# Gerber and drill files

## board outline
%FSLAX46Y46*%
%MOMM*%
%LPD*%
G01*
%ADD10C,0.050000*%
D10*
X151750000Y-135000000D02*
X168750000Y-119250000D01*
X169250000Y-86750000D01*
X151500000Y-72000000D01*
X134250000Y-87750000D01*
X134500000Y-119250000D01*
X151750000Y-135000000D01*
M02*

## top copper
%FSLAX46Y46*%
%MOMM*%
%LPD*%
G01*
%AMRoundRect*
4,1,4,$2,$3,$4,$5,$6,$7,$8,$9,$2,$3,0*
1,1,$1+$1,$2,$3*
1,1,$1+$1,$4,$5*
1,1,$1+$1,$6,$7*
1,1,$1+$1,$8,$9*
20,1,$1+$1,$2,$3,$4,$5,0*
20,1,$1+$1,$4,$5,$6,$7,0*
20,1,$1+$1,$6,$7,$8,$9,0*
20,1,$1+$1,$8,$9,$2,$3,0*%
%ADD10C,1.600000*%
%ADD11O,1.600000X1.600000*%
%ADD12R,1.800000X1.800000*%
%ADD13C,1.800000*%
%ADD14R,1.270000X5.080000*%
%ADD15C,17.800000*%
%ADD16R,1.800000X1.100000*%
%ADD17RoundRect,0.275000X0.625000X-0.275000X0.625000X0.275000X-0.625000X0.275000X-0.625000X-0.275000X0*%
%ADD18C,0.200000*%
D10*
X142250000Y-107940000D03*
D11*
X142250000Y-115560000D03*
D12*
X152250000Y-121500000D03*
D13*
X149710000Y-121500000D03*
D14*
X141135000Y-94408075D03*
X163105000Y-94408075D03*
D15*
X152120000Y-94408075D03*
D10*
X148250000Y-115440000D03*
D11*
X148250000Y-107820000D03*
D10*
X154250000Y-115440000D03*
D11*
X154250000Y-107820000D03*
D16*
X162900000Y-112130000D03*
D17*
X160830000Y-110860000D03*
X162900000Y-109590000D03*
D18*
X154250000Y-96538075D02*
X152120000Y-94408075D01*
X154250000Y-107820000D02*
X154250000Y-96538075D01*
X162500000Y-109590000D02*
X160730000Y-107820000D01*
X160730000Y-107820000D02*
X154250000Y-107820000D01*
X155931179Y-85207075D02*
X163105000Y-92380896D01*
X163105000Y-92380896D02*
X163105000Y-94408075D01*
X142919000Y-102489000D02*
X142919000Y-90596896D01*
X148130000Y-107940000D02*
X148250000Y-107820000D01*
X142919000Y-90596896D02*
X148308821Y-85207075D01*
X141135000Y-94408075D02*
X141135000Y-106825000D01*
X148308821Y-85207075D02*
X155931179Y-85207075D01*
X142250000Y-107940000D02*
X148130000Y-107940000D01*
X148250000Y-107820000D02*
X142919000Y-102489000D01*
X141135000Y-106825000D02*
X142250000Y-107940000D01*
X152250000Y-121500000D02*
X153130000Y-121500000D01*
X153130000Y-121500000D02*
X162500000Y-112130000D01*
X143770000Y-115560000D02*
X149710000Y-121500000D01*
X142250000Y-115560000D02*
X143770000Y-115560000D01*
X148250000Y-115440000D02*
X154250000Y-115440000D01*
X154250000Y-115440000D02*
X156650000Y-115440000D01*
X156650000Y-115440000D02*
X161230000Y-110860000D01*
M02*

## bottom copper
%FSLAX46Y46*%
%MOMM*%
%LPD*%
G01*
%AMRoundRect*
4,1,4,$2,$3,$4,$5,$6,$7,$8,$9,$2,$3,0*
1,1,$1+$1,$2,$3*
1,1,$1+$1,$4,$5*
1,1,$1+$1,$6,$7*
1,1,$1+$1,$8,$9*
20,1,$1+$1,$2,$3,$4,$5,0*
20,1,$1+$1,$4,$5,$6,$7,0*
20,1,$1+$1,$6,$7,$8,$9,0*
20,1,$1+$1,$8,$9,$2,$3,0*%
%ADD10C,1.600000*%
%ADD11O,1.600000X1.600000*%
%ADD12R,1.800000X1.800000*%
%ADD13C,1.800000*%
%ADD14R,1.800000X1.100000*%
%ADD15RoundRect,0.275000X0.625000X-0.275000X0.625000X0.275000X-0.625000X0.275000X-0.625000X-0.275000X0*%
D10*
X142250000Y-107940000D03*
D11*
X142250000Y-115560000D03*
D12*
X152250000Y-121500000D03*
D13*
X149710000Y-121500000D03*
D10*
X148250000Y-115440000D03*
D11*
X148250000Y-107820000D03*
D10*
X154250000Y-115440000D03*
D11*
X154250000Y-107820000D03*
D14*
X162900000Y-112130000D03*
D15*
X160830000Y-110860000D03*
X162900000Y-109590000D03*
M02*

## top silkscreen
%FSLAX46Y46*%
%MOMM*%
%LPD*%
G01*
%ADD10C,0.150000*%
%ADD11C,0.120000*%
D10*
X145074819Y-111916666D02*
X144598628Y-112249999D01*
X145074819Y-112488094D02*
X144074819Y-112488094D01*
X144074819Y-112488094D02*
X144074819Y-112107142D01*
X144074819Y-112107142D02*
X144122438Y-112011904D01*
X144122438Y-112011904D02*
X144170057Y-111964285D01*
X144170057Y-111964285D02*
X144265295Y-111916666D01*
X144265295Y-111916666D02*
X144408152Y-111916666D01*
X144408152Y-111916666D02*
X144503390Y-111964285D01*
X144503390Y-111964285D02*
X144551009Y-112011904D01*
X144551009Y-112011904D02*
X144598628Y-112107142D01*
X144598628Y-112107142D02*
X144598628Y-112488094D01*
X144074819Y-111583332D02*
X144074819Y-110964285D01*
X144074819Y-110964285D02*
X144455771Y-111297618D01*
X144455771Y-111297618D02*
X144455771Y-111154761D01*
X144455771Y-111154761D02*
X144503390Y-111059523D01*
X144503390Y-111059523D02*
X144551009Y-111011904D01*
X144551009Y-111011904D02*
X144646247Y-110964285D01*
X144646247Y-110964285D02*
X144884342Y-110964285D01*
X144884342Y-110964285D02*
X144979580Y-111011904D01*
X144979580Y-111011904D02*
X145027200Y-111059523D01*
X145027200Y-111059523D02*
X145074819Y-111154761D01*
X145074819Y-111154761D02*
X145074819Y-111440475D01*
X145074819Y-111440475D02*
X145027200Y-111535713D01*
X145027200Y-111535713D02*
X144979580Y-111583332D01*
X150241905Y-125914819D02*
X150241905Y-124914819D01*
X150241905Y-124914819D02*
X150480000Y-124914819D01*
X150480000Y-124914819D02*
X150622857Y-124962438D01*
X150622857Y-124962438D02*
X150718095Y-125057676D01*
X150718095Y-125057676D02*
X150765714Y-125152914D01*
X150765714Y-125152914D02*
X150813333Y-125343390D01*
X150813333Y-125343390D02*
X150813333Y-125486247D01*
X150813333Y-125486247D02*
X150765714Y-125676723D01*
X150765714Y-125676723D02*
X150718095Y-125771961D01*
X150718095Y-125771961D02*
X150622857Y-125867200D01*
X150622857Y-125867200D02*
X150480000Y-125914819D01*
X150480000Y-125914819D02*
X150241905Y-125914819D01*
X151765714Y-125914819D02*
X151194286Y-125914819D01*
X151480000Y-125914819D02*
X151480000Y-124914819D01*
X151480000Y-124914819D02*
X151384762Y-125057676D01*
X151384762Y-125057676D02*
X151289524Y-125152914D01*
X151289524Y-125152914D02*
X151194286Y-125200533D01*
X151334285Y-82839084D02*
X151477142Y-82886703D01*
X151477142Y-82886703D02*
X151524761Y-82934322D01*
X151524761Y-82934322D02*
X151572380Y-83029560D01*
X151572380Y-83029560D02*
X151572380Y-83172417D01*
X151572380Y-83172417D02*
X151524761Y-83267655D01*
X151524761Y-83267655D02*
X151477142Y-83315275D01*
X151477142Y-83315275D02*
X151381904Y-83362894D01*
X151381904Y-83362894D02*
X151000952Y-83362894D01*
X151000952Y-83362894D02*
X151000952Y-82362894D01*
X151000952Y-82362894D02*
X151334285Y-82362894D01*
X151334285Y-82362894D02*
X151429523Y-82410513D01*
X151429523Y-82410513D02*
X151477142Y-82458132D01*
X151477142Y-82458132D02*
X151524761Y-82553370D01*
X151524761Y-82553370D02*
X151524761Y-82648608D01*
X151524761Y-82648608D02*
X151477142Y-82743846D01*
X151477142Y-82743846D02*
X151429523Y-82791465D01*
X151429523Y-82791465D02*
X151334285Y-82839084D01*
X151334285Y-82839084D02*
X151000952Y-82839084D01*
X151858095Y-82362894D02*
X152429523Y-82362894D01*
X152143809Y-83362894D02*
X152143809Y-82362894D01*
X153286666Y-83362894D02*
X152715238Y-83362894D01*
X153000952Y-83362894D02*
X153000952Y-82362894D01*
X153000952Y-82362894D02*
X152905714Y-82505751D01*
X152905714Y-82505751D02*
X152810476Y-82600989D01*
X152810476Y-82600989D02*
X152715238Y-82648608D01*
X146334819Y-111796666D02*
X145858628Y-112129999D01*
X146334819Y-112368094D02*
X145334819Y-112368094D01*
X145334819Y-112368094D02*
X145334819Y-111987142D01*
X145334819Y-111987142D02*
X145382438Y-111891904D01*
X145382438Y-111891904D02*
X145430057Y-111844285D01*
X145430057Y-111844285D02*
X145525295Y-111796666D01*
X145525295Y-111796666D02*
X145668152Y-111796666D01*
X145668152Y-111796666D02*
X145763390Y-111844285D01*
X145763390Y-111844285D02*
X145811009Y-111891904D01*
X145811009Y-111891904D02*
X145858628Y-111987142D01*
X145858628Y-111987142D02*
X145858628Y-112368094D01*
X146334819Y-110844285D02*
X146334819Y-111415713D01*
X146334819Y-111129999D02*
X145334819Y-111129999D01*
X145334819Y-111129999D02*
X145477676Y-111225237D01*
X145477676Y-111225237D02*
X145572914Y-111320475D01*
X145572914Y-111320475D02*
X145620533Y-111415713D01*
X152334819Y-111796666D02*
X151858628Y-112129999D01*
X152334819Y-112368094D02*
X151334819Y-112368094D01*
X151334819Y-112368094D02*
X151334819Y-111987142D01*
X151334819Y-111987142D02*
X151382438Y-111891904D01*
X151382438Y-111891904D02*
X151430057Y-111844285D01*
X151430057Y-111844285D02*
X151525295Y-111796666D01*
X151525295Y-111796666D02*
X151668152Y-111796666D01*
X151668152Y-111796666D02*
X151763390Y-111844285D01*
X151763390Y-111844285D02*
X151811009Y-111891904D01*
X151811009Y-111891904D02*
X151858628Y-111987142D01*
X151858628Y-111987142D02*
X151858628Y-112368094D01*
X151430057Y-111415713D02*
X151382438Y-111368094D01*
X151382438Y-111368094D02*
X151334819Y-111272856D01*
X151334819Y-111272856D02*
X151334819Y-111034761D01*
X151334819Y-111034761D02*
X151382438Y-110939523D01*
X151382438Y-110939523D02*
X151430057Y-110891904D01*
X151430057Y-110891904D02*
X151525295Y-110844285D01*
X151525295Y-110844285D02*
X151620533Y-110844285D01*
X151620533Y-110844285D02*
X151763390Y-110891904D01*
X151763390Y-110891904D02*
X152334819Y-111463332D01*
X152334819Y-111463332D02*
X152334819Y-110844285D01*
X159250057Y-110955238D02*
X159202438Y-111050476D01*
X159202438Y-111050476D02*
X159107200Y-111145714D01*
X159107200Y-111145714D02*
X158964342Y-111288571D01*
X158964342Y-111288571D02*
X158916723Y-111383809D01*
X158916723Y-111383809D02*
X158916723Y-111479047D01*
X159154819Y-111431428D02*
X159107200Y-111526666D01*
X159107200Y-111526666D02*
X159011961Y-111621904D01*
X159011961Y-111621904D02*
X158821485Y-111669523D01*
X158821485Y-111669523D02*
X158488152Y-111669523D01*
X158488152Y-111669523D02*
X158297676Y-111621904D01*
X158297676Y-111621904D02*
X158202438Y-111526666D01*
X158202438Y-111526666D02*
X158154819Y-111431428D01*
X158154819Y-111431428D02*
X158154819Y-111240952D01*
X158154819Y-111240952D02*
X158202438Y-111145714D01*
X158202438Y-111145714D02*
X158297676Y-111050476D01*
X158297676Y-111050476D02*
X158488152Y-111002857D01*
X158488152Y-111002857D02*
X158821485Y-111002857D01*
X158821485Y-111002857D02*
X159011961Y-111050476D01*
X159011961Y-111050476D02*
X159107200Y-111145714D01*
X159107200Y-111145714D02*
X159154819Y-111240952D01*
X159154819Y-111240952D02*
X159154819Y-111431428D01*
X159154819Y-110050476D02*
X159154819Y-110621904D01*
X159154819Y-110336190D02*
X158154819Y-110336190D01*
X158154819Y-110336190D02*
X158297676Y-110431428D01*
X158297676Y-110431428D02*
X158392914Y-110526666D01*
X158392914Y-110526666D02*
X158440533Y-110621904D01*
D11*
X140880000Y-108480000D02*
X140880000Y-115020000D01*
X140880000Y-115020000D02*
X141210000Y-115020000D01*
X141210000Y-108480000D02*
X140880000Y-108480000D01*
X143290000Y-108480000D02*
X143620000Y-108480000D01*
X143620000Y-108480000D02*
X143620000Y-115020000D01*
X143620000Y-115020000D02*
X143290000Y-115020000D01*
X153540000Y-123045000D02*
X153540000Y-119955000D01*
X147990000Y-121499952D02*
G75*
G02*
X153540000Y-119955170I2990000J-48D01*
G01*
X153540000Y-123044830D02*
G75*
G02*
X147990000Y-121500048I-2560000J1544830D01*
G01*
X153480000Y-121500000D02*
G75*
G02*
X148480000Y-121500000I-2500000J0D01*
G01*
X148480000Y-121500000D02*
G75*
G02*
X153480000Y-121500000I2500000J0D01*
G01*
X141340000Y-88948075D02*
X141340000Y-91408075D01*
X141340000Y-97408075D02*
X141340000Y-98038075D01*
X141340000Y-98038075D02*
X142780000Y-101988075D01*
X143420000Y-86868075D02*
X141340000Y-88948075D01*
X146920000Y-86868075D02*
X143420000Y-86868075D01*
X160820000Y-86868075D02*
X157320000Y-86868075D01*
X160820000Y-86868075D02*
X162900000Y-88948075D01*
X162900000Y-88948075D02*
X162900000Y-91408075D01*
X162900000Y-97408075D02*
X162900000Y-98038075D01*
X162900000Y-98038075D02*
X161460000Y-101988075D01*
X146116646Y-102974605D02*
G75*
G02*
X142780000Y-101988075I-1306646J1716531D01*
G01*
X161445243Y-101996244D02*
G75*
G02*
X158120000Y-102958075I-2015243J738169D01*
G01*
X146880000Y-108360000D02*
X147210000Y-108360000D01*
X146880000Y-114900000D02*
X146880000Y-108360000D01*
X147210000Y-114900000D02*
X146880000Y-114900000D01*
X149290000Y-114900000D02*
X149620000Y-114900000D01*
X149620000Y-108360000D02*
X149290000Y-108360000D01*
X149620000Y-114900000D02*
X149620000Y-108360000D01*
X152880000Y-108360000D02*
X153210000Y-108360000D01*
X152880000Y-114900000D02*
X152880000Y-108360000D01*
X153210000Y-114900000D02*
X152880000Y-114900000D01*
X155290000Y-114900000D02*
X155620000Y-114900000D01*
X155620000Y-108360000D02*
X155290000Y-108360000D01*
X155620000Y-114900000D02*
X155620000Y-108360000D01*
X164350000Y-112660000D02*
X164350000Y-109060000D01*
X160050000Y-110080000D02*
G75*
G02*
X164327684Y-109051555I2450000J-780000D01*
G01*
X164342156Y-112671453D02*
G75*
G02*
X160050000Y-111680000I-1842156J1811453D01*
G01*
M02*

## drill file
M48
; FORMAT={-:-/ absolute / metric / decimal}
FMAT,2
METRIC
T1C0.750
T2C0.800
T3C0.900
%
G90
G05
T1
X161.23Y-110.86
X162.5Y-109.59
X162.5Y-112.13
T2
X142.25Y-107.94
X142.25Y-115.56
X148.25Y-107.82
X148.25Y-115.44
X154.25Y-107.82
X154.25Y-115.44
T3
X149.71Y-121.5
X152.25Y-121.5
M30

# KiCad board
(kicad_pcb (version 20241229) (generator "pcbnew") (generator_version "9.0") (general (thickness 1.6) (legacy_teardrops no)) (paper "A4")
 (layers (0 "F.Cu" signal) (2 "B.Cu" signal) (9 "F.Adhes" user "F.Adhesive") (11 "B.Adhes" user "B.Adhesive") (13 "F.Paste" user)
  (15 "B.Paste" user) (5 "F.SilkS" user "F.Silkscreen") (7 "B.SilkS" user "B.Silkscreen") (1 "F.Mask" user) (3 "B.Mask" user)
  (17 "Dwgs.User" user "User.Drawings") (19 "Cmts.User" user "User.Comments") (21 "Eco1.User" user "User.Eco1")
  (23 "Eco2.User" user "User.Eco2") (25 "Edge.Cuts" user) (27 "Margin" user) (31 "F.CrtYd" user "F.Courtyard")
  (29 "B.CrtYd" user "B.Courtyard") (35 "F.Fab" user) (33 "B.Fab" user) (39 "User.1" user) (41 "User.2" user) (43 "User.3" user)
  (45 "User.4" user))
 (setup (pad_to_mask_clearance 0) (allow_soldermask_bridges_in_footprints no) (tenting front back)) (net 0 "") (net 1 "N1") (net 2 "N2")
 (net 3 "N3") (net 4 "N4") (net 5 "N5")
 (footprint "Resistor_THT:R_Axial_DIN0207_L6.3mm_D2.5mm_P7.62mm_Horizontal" (layer "F.Cu") (at 142.25 107.94 -90)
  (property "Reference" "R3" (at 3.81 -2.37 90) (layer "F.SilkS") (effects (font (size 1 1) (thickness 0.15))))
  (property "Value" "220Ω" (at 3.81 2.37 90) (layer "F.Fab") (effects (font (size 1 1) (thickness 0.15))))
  (fp_line (start 0.54 1.37) (end 7.08 1.37) (stroke (width 0.12) (type solid)) (layer "F.SilkS"))
  (fp_line (start 7.08 1.37) (end 7.08 1.04) (stroke (width 0.12) (type solid)) (layer "F.SilkS"))
  (fp_line (start 0.54 1.04) (end 0.54 1.37) (stroke (width 0.12) (type solid)) (layer "F.SilkS"))
  (fp_line (start 0.54 -1.04) (end 0.54 -1.37) (stroke (width 0.12) (type solid)) (layer "F.SilkS"))
  (fp_line (start 0.54 -1.37) (end 7.08 -1.37) (stroke (width 0.12) (type solid)) (layer "F.SilkS"))
  (fp_line (start 7.08 -1.37) (end 7.08 -1.04) (stroke (width 0.12) (type solid)) (layer "F.SilkS"))
  (pad "1" thru_hole circle (at 0 0 270) (size 1.6 1.6) (drill 0.8) (layers "*.Cu" "*.Mask") (remove_unused_layers no) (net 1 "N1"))
  (pad "2" thru_hole oval (at 7.62 0 270) (size 1.6 1.6) (drill 0.8) (layers "*.Cu" "*.Mask") (remove_unused_layers no) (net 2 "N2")))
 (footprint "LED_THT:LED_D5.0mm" (layer "F.Cu") (at 152.25 121.5 180)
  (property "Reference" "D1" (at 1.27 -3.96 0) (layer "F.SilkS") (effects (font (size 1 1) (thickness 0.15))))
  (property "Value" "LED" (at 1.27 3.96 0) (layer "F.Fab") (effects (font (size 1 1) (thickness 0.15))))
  (fp_line (start -1.29 -1.545) (end -1.29 1.545) (stroke (width 0.12) (type solid)) (layer "F.SilkS"))
  (fp_arc (start 4.26 0.000048) (mid 2.071756 2.880501) (end -1.29 1.54483) (stroke (width 0.12) (type solid)) (layer "F.SilkS"))
  (fp_arc (start -1.29 -1.54483) (mid 2.071756 -2.880501) (end 4.26 -0.000048) (stroke (width 0.12) (type solid)) (layer "F.SilkS"))
  (fp_circle (center 1.27 0) (end 3.77 0) (stroke (width 0.12) (type solid)) (fill no) (layer "F.SilkS"))
  (pad "1" thru_hole rect (at 0 0 180) (size 1.8 1.8) (drill 0.9) (layers "*.Cu" "*.Mask") (remove_unused_layers no) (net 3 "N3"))
  (pad "2" thru_hole circle (at 2.54 0 180) (size 1.8 1.8) (drill 0.9) (layers "*.Cu" "*.Mask") (remove_unused_layers no) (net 2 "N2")))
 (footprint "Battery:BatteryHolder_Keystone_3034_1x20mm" (layer "F.Cu") (at 152.12 94.408075)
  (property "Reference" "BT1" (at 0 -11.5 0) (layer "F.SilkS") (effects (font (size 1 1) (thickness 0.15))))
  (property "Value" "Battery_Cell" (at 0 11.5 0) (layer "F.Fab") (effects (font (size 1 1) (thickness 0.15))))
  (fp_line (start -10.78 -5.46) (end -10.78 -3) (stroke (width 0.12) (type solid)) (layer "F.SilkS"))
  (fp_line (start -10.78 3) (end -10.78 3.63) (stroke (width 0.12) (type solid)) (layer "F.SilkS"))
  (fp_line (start -10.78 3.63) (end -9.34 7.58) (stroke (width 0.12) (type solid)) (layer "F.SilkS"))
  (fp_line (start -8.7 -7.54) (end -10.78 -5.46) (stroke (width 0.12) (type solid)) (layer "F.SilkS"))
  (fp_line (start -5.2 -7.54) (end -8.7 -7.54) (stroke (width 0.12) (type solid)) (layer "F.SilkS"))
  (fp_line (start 8.7 -7.54) (end 5.2 -7.54) (stroke (width 0.12) (type solid)) (layer "F.SilkS"))
  (fp_line (start 8.7 -7.54) (end 10.78 -5.46) (stroke (width 0.12) (type solid)) (layer "F.SilkS"))
  (fp_line (start 10.78 -5.46) (end 10.78 -3) (stroke (width 0.12) (type solid)) (layer "F.SilkS"))
  (fp_line (start 10.78 3) (end 10.78 3.63) (stroke (width 0.12) (type solid)) (layer "F.SilkS"))
  (fp_line (start 10.78 3.63) (end 9.34 7.58) (stroke (width 0.12) (type solid)) (layer "F.SilkS"))
  (fp_arc (start -6.003354 8.56653) (mid -7.921654 8.918738) (end -9.34 7.58) (stroke (width 0.12) (type solid)) (layer "F.SilkS"))
  (fp_arc (start 9.325243 7.588169) (mid 7.90634 8.911668) (end 6 8.55) (stroke (width 0.12) (type solid)) (layer "F.SilkS"))
  (pad "1" smd rect (at -10.985 0) (size 1.27 5.08) (layers "F.Cu" "F.Mask" "F.Paste") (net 1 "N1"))
  (pad "1" smd rect (at 10.985 0) (size 1.27 5.08) (layers "F.Cu" "F.Mask" "F.Paste") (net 1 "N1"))
  (pad "2" smd circle (at 0 0) (size 17.8 17.8) (layers "F.Cu" "F.Mask") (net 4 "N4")))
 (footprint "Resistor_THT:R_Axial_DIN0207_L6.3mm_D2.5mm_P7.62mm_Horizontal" (layer "F.Cu") (at 148.25 115.44 90)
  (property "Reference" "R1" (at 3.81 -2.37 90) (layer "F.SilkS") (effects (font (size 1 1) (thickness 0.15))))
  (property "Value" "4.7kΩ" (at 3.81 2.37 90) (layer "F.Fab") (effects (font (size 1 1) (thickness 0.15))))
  (fp_line (start 7.08 -1.37) (end 7.08 -1.04) (stroke (width 0.12) (type solid)) (layer "F.SilkS"))
  (fp_line (start 0.54 -1.37) (end 7.08 -1.37) (stroke (width 0.12) (type solid)) (layer "F.SilkS"))
  (fp_line (start 0.54 -1.04) (end 0.54 -1.37) (stroke (width 0.12) (type solid)) (layer "F.SilkS"))
  (fp_line (start 0.54 1.04) (end 0.54 1.37) (stroke (width 0.12) (type solid)) (layer "F.SilkS"))
  (fp_line (start 7.08 1.37) (end 7.08 1.04) (stroke (width 0.12) (type solid)) (layer "F.SilkS"))
  (fp_line (start 0.54 1.37) (end 7.08 1.37) (stroke (width 0.12) (type solid)) (layer "F.SilkS"))
  (pad "1" thru_hole circle (at 0 0 90) (size 1.6 1.6) (drill 0.8) (layers "*.Cu" "*.Mask") (remove_unused_layers no) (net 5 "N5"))
  (pad "2" thru_hole oval (at 7.62 0 90) (size 1.6 1.6) (drill 0.8) (layers "*.Cu" "*.Mask") (remove_unused_layers no) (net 1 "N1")))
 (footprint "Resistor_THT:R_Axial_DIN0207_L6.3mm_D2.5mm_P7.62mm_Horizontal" (layer "F.Cu") (at 154.25 115.44 90)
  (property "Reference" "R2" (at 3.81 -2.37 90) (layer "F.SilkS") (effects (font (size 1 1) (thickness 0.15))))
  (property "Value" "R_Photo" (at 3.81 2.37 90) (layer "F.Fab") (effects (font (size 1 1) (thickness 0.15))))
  (fp_line (start 7.08 -1.37) (end 7.08 -1.04) (stroke (width 0.12) (type solid)) (layer "F.SilkS"))
  (fp_line (start 0.54 -1.37) (end 7.08 -1.37) (stroke (width 0.12) (type solid)) (layer "F.SilkS"))
  (fp_line (start 0.54 -1.04) (end 0.54 -1.37) (stroke (width 0.12) (type solid)) (layer "F.SilkS"))
  (fp_line (start 0.54 1.04) (end 0.54 1.37) (stroke (width 0.12) (type solid)) (layer "F.SilkS"))
  (fp_line (start 7.08 1.37) (end 7.08 1.04) (stroke (width 0.12) (type solid)) (layer "F.SilkS"))
  (fp_line (start 0.54 1.37) (end 7.08 1.37) (stroke (width 0.12) (type solid)) (layer "F.SilkS"))
  (pad "1" thru_hole circle (at 0 0 90) (size 1.6 1.6) (drill 0.8) (layers "*.Cu" "*.Mask") (remove_unused_layers no) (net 5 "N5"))
  (pad "2" thru_hole oval (at 7.62 0 90) (size 1.6 1.6) (drill 0.8) (layers "*.Cu" "*.Mask") (remove_unused_layers no) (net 4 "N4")))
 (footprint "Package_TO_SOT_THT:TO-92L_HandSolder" (layer "F.Cu") (at 162.5 112.13 90)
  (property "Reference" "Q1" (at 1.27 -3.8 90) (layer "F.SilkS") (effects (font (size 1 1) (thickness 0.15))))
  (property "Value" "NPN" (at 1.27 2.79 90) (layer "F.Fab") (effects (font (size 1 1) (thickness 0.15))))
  (fp_line (start -0.53 1.85) (end 3.07 1.85) (stroke (width 0.12) (type solid)) (layer "F.SilkS"))
  (fp_arc (start 2.05 -2.45) (mid 3.769931 -0.601036) (end 3.078445 1.827684) (stroke (width 0.12) (type solid)) (layer "F.SilkS"))
  (fp_arc (start -0.541453 1.842156) (mid -1.247298 -0.581475) (end 0.45 -2.45) (stroke (width 0.12) (type solid)) (layer "F.SilkS"))
  (pad "1" thru_hole rect (at 0 0 90) (size 1.1 1.8) (drill 0.75 (offset 0 0.4)) (layers "*.Cu" "*.Mask") (remove_unused_layers no)
   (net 3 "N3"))
  (pad "2" thru_hole roundrect (at 1.27 -1.27 90) (size 1.1 1.8) (drill 0.75 (offset 0 -0.4)) (layers "*.Cu" "*.Mask")
   (remove_unused_layers no) (roundrect_rratio 0.25) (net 5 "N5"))
  (pad "3" thru_hole roundrect (at 2.54 0 90) (size 1.1 1.8) (drill 0.75 (offset 0 0.4)) (layers "*.Cu" "*.Mask") (remove_unused_layers no)
   (roundrect_rratio 0.25) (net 4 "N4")))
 (gr_poly
  (pts (xy 151.75 135) (xy 168.75 119.25) (xy 169.25 86.75) (xy 151.5 72) (xy 134.25 87.75) (xy 134.5 119.25))
  (stroke (width 0.05) (type solid)) (fill no) (layer "Edge.Cuts"))
 (segment (start 154.25 96.538075) (end 152.12 94.408075) (width 0.2) (layer "F.Cu") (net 4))
 (segment (start 154.25 107.82) (end 154.25 96.538075) (width 0.2) (layer "F.Cu") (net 4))
 (segment (start 162.5 109.59) (end 160.73 107.82) (width 0.2) (layer "F.Cu") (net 4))
 (segment (start 160.73 107.82) (end 154.25 107.82) (width 0.2) (layer "F.Cu") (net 4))
 (segment (start 155.931179 85.207075) (end 163.105 92.380896) (width 0.2) (layer "F.Cu") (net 1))
 (segment (start 163.105 92.380896) (end 163.105 94.408075) (width 0.2) (layer "F.Cu") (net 1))
 (segment (start 142.919 102.489) (end 142.919 90.596896) (width 0.2) (layer "F.Cu") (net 1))
 (segment (start 148.13 107.94) (end 148.25 107.82) (width 0.2) (layer "F.Cu") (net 1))
 (segment (start 142.919 90.596896) (end 148.308821 85.207075) (width 0.2) (layer "F.Cu") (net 1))
 (segment (start 141.135 94.408075) (end 141.135 106.825) (width 0.2) (layer "F.Cu") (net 1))
 (segment (start 148.308821 85.207075) (end 155.931179 85.207075) (width 0.2) (layer "F.Cu") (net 1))
 (segment (start 142.25 107.94) (end 148.13 107.94) (width 0.2) (layer "F.Cu") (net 1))
 (segment (start 148.25 107.82) (end 142.919 102.489) (width 0.2) (layer "F.Cu") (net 1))
 (segment (start 141.135 106.825) (end 142.25 107.94) (width 0.2) (layer "F.Cu") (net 1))
 (segment (start 152.25 121.5) (end 153.13 121.5) (width 0.2) (layer "F.Cu") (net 3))
 (segment (start 153.13 121.5) (end 162.5 112.13) (width 0.2) (layer "F.Cu") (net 3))
 (segment (start 143.77 115.56) (end 149.71 121.5) (width 0.2) (layer "F.Cu") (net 2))
 (segment (start 142.25 115.56) (end 143.77 115.56) (width 0.2) (layer "F.Cu") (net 2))
 (segment (start 148.25 115.44) (end 154.25 115.44) (width 0.2) (layer "F.Cu") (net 5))
 (segment (start 154.25 115.44) (end 156.65 115.44) (width 0.2) (layer "F.Cu") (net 5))
 (segment (start 156.65 115.44) (end 161.23 110.86) (width 0.2) (layer "F.Cu") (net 5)))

